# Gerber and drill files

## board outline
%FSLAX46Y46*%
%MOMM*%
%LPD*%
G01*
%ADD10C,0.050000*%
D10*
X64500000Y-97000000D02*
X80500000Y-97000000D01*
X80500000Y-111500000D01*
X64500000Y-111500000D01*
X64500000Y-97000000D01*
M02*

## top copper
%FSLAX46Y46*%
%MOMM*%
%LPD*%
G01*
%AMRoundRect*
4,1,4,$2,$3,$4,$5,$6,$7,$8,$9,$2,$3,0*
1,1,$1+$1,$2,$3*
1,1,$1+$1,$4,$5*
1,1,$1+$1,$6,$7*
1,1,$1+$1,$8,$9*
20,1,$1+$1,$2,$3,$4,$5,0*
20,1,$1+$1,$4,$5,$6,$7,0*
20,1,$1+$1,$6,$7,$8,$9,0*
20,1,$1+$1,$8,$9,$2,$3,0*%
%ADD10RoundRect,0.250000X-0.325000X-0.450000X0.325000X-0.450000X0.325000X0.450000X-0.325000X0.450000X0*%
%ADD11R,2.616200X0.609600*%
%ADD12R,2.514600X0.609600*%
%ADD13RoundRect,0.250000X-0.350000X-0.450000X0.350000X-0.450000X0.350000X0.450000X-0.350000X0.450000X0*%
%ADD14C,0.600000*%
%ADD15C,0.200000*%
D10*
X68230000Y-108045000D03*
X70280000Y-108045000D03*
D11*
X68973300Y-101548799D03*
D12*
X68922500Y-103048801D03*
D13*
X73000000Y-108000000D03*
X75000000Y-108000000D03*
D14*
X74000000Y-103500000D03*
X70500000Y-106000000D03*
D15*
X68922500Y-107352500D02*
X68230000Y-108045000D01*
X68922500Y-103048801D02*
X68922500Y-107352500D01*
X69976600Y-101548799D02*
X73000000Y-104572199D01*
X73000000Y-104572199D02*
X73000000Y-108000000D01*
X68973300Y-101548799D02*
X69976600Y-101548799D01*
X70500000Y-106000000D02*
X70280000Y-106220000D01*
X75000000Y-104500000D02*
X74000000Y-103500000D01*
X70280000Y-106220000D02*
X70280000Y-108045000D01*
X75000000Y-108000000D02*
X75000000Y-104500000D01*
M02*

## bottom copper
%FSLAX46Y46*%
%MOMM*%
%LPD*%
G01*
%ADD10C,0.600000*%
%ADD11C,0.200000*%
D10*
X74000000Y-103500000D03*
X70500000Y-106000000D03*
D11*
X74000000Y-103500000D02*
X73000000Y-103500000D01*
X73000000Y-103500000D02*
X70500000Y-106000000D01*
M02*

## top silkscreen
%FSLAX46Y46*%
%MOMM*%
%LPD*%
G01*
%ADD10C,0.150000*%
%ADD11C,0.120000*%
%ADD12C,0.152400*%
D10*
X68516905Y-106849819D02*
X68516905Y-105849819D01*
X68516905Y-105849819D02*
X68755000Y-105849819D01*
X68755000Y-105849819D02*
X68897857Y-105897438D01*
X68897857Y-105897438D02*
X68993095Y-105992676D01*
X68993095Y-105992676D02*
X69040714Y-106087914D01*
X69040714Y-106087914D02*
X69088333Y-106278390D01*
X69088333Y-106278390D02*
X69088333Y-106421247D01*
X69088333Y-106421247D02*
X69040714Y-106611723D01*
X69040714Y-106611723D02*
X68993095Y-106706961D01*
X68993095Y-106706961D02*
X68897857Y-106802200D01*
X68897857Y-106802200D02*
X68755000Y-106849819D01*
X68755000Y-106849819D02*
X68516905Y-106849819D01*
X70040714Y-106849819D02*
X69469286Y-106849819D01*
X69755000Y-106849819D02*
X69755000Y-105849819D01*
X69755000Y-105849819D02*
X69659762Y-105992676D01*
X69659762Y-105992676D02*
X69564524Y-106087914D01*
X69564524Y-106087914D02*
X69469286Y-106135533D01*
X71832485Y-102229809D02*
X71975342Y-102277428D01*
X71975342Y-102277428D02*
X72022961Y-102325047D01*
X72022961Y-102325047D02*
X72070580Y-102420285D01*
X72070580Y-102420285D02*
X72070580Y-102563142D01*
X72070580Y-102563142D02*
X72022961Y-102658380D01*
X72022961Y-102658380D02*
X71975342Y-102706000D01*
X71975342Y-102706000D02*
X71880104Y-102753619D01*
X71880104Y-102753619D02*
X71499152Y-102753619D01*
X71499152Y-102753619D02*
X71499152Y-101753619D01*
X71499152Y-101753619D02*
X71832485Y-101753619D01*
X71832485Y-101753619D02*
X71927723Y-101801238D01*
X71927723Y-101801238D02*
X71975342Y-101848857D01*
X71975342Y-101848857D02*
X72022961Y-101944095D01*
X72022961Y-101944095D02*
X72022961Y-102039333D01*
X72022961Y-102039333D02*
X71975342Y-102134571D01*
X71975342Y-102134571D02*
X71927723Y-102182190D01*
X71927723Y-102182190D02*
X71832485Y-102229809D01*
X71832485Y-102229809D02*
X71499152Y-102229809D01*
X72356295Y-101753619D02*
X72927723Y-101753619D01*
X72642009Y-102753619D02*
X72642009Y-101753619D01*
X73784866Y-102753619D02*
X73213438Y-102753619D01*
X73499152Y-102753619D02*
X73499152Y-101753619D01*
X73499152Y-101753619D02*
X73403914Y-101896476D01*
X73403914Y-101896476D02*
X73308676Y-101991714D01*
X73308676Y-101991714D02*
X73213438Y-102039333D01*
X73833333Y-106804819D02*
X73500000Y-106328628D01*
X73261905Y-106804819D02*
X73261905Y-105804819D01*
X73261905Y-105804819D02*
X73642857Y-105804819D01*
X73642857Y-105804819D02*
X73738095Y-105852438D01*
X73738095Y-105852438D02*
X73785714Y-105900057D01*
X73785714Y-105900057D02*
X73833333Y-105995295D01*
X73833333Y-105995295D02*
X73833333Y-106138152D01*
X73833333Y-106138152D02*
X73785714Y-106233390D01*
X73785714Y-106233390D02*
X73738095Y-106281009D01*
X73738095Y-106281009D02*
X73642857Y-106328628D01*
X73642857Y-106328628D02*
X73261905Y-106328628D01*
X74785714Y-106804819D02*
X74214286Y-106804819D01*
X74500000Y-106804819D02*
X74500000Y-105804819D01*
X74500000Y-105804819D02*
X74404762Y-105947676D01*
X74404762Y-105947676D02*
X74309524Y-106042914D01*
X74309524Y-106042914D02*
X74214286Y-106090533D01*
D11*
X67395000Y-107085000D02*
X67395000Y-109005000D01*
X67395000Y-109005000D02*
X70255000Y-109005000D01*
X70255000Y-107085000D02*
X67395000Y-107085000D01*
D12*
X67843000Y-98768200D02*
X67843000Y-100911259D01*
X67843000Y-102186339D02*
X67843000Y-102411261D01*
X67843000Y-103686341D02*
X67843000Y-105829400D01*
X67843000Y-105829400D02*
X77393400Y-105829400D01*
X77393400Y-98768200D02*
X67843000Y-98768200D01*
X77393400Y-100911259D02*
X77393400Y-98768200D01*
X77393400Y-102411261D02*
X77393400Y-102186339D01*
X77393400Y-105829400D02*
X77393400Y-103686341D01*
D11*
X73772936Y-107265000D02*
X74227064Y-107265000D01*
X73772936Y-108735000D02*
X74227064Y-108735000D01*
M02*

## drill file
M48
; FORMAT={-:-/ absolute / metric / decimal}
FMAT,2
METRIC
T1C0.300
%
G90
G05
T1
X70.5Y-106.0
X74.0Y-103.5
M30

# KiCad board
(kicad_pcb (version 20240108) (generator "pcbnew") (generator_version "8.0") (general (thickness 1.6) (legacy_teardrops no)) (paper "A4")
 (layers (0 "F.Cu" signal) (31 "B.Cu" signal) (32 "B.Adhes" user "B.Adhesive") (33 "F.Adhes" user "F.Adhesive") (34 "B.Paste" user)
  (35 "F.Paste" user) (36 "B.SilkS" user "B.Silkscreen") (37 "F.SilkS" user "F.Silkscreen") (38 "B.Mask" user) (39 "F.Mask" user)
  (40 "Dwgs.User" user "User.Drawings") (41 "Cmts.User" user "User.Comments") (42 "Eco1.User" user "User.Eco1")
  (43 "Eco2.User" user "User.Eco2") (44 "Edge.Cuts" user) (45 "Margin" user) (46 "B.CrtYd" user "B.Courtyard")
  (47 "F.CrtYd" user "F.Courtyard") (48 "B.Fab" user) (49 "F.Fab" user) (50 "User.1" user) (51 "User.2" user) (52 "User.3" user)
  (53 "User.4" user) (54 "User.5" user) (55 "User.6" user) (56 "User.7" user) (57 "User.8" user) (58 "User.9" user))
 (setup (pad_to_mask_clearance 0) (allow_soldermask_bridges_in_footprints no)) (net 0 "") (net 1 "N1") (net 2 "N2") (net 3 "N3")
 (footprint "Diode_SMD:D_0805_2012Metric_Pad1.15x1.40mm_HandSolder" (layer "F.Cu") (at 69.255 108.045)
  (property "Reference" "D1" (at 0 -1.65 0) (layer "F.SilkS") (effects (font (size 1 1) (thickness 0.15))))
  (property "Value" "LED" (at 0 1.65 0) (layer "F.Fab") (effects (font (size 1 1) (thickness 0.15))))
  (fp_line (start -1.86 -0.96) (end -1.86 0.96) (stroke (width 0.12) (type solid)) (layer "F.SilkS"))
  (fp_line (start -1.86 0.96) (end 1 0.96) (stroke (width 0.12) (type solid)) (layer "F.SilkS"))
  (fp_line (start 1 -0.96) (end -1.86 -0.96) (stroke (width 0.12) (type solid)) (layer "F.SilkS"))
  (pad "1" smd roundrect (at -1.025 0) (size 1.15 1.4) (layers "F.Cu" "F.Paste" "F.Mask") (roundrect_rratio 0.217391) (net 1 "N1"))
  (pad "2" smd roundrect (at 1.025 0) (size 1.15 1.4) (layers "F.Cu" "F.Paste" "F.Mask") (roundrect_rratio 0.217391) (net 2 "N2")))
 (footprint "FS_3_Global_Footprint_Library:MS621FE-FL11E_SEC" (layer "F.Cu") (at 72.6182 102.2988)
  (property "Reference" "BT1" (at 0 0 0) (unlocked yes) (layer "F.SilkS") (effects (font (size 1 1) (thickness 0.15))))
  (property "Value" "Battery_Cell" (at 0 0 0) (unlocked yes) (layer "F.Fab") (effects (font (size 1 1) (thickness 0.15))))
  (fp_line (start -4.7752 -3.5306) (end -4.7752 -1.387541) (stroke (width 0.1524) (type solid)) (layer "F.SilkS"))
  (fp_line (start -4.7752 -0.112461) (end -4.7752 0.112461) (stroke (width 0.1524) (type solid)) (layer "F.SilkS"))
  (fp_line (start -4.7752 1.387541) (end -4.7752 3.5306) (stroke (width 0.1524) (type solid)) (layer "F.SilkS"))
  (fp_line (start -4.7752 3.5306) (end 4.7752 3.5306) (stroke (width 0.1524) (type solid)) (layer "F.SilkS"))
  (fp_line (start 4.7752 -3.5306) (end -4.7752 -3.5306) (stroke (width 0.1524) (type solid)) (layer "F.SilkS"))
  (fp_line (start 4.7752 -1.387541) (end 4.7752 -3.5306) (stroke (width 0.1524) (type solid)) (layer "F.SilkS"))
  (fp_line (start 4.7752 0.112461) (end 4.7752 -0.112461) (stroke (width 0.1524) (type solid)) (layer "F.SilkS"))
  (fp_line (start 4.7752 3.5306) (end 4.7752 1.387541) (stroke (width 0.1524) (type solid)) (layer "F.SilkS"))
  (pad "1" smd rect (at -3.6449 -0.750001) (size 2.6162 0.6096) (layers "F.Cu" "F.Paste" "F.Mask") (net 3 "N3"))
  (pad "2" smd rect (at -3.6957 0.750001) (size 2.5146 0.6096) (layers "F.Cu" "F.Paste" "F.Mask") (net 1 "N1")))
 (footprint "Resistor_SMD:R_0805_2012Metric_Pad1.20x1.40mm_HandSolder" (layer "F.Cu") (at 74 108)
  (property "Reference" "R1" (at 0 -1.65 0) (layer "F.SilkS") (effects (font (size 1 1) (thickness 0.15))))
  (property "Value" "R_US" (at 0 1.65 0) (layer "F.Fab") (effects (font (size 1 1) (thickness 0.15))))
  (fp_line (start -0.227064 -0.735) (end 0.227064 -0.735) (stroke (width 0.12) (type solid)) (layer "F.SilkS"))
  (fp_line (start -0.227064 0.735) (end 0.227064 0.735) (stroke (width 0.12) (type solid)) (layer "F.SilkS"))
  (pad "1" smd roundrect (at -1 0) (size 1.2 1.4) (layers "F.Cu" "F.Paste" "F.Mask") (roundrect_rratio 0.208333) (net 3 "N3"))
  (pad "2" smd roundrect (at 1 0) (size 1.2 1.4) (layers "F.Cu" "F.Paste" "F.Mask") (roundrect_rratio 0.208333) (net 2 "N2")))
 (gr_rect (start 64.5 97) (end 80.5 111.5) (stroke (width 0.05) (type default)) (fill none) (layer "Edge.Cuts"))
 (segment (start 68.9225 107.3525) (end 68.23 108.045) (width 0.2) (layer "F.Cu") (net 1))
 (segment (start 68.9225 103.048801) (end 68.9225 107.3525) (width 0.2) (layer "F.Cu") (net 1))
 (segment (start 69.9766 101.548799) (end 73 104.572199) (width 0.2) (layer "F.Cu") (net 3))
 (segment (start 73 104.572199) (end 73 108) (width 0.2) (layer "F.Cu") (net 3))
 (segment (start 68.9733 101.548799) (end 69.9766 101.548799) (width 0.2) (layer "F.Cu") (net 3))
 (segment (start 70.5 106) (end 70.28 106.22) (width 0.2) (layer "F.Cu") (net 2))
 (segment (start 75 104.5) (end 74 103.5) (width 0.2) (layer "F.Cu") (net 2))
 (segment (start 70.28 106.22) (end 70.28 108.045) (width 0.2) (layer "F.Cu") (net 2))
 (segment (start 75 108) (end 75 104.5) (width 0.2) (layer "F.Cu") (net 2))
 (via (at 74 103.5) (size 0.6) (drill 0.3) (layers "F.Cu" "B.Cu") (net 2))
 (via (at 70.5 106) (size 0.6) (drill 0.3) (layers "F.Cu" "B.Cu") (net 2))
 (segment (start 74 103.5) (end 73 103.5) (width 0.2) (layer "B.Cu") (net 2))
 (segment (start 73 103.5) (end 70.5 106) (width 0.2) (layer "B.Cu") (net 2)))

